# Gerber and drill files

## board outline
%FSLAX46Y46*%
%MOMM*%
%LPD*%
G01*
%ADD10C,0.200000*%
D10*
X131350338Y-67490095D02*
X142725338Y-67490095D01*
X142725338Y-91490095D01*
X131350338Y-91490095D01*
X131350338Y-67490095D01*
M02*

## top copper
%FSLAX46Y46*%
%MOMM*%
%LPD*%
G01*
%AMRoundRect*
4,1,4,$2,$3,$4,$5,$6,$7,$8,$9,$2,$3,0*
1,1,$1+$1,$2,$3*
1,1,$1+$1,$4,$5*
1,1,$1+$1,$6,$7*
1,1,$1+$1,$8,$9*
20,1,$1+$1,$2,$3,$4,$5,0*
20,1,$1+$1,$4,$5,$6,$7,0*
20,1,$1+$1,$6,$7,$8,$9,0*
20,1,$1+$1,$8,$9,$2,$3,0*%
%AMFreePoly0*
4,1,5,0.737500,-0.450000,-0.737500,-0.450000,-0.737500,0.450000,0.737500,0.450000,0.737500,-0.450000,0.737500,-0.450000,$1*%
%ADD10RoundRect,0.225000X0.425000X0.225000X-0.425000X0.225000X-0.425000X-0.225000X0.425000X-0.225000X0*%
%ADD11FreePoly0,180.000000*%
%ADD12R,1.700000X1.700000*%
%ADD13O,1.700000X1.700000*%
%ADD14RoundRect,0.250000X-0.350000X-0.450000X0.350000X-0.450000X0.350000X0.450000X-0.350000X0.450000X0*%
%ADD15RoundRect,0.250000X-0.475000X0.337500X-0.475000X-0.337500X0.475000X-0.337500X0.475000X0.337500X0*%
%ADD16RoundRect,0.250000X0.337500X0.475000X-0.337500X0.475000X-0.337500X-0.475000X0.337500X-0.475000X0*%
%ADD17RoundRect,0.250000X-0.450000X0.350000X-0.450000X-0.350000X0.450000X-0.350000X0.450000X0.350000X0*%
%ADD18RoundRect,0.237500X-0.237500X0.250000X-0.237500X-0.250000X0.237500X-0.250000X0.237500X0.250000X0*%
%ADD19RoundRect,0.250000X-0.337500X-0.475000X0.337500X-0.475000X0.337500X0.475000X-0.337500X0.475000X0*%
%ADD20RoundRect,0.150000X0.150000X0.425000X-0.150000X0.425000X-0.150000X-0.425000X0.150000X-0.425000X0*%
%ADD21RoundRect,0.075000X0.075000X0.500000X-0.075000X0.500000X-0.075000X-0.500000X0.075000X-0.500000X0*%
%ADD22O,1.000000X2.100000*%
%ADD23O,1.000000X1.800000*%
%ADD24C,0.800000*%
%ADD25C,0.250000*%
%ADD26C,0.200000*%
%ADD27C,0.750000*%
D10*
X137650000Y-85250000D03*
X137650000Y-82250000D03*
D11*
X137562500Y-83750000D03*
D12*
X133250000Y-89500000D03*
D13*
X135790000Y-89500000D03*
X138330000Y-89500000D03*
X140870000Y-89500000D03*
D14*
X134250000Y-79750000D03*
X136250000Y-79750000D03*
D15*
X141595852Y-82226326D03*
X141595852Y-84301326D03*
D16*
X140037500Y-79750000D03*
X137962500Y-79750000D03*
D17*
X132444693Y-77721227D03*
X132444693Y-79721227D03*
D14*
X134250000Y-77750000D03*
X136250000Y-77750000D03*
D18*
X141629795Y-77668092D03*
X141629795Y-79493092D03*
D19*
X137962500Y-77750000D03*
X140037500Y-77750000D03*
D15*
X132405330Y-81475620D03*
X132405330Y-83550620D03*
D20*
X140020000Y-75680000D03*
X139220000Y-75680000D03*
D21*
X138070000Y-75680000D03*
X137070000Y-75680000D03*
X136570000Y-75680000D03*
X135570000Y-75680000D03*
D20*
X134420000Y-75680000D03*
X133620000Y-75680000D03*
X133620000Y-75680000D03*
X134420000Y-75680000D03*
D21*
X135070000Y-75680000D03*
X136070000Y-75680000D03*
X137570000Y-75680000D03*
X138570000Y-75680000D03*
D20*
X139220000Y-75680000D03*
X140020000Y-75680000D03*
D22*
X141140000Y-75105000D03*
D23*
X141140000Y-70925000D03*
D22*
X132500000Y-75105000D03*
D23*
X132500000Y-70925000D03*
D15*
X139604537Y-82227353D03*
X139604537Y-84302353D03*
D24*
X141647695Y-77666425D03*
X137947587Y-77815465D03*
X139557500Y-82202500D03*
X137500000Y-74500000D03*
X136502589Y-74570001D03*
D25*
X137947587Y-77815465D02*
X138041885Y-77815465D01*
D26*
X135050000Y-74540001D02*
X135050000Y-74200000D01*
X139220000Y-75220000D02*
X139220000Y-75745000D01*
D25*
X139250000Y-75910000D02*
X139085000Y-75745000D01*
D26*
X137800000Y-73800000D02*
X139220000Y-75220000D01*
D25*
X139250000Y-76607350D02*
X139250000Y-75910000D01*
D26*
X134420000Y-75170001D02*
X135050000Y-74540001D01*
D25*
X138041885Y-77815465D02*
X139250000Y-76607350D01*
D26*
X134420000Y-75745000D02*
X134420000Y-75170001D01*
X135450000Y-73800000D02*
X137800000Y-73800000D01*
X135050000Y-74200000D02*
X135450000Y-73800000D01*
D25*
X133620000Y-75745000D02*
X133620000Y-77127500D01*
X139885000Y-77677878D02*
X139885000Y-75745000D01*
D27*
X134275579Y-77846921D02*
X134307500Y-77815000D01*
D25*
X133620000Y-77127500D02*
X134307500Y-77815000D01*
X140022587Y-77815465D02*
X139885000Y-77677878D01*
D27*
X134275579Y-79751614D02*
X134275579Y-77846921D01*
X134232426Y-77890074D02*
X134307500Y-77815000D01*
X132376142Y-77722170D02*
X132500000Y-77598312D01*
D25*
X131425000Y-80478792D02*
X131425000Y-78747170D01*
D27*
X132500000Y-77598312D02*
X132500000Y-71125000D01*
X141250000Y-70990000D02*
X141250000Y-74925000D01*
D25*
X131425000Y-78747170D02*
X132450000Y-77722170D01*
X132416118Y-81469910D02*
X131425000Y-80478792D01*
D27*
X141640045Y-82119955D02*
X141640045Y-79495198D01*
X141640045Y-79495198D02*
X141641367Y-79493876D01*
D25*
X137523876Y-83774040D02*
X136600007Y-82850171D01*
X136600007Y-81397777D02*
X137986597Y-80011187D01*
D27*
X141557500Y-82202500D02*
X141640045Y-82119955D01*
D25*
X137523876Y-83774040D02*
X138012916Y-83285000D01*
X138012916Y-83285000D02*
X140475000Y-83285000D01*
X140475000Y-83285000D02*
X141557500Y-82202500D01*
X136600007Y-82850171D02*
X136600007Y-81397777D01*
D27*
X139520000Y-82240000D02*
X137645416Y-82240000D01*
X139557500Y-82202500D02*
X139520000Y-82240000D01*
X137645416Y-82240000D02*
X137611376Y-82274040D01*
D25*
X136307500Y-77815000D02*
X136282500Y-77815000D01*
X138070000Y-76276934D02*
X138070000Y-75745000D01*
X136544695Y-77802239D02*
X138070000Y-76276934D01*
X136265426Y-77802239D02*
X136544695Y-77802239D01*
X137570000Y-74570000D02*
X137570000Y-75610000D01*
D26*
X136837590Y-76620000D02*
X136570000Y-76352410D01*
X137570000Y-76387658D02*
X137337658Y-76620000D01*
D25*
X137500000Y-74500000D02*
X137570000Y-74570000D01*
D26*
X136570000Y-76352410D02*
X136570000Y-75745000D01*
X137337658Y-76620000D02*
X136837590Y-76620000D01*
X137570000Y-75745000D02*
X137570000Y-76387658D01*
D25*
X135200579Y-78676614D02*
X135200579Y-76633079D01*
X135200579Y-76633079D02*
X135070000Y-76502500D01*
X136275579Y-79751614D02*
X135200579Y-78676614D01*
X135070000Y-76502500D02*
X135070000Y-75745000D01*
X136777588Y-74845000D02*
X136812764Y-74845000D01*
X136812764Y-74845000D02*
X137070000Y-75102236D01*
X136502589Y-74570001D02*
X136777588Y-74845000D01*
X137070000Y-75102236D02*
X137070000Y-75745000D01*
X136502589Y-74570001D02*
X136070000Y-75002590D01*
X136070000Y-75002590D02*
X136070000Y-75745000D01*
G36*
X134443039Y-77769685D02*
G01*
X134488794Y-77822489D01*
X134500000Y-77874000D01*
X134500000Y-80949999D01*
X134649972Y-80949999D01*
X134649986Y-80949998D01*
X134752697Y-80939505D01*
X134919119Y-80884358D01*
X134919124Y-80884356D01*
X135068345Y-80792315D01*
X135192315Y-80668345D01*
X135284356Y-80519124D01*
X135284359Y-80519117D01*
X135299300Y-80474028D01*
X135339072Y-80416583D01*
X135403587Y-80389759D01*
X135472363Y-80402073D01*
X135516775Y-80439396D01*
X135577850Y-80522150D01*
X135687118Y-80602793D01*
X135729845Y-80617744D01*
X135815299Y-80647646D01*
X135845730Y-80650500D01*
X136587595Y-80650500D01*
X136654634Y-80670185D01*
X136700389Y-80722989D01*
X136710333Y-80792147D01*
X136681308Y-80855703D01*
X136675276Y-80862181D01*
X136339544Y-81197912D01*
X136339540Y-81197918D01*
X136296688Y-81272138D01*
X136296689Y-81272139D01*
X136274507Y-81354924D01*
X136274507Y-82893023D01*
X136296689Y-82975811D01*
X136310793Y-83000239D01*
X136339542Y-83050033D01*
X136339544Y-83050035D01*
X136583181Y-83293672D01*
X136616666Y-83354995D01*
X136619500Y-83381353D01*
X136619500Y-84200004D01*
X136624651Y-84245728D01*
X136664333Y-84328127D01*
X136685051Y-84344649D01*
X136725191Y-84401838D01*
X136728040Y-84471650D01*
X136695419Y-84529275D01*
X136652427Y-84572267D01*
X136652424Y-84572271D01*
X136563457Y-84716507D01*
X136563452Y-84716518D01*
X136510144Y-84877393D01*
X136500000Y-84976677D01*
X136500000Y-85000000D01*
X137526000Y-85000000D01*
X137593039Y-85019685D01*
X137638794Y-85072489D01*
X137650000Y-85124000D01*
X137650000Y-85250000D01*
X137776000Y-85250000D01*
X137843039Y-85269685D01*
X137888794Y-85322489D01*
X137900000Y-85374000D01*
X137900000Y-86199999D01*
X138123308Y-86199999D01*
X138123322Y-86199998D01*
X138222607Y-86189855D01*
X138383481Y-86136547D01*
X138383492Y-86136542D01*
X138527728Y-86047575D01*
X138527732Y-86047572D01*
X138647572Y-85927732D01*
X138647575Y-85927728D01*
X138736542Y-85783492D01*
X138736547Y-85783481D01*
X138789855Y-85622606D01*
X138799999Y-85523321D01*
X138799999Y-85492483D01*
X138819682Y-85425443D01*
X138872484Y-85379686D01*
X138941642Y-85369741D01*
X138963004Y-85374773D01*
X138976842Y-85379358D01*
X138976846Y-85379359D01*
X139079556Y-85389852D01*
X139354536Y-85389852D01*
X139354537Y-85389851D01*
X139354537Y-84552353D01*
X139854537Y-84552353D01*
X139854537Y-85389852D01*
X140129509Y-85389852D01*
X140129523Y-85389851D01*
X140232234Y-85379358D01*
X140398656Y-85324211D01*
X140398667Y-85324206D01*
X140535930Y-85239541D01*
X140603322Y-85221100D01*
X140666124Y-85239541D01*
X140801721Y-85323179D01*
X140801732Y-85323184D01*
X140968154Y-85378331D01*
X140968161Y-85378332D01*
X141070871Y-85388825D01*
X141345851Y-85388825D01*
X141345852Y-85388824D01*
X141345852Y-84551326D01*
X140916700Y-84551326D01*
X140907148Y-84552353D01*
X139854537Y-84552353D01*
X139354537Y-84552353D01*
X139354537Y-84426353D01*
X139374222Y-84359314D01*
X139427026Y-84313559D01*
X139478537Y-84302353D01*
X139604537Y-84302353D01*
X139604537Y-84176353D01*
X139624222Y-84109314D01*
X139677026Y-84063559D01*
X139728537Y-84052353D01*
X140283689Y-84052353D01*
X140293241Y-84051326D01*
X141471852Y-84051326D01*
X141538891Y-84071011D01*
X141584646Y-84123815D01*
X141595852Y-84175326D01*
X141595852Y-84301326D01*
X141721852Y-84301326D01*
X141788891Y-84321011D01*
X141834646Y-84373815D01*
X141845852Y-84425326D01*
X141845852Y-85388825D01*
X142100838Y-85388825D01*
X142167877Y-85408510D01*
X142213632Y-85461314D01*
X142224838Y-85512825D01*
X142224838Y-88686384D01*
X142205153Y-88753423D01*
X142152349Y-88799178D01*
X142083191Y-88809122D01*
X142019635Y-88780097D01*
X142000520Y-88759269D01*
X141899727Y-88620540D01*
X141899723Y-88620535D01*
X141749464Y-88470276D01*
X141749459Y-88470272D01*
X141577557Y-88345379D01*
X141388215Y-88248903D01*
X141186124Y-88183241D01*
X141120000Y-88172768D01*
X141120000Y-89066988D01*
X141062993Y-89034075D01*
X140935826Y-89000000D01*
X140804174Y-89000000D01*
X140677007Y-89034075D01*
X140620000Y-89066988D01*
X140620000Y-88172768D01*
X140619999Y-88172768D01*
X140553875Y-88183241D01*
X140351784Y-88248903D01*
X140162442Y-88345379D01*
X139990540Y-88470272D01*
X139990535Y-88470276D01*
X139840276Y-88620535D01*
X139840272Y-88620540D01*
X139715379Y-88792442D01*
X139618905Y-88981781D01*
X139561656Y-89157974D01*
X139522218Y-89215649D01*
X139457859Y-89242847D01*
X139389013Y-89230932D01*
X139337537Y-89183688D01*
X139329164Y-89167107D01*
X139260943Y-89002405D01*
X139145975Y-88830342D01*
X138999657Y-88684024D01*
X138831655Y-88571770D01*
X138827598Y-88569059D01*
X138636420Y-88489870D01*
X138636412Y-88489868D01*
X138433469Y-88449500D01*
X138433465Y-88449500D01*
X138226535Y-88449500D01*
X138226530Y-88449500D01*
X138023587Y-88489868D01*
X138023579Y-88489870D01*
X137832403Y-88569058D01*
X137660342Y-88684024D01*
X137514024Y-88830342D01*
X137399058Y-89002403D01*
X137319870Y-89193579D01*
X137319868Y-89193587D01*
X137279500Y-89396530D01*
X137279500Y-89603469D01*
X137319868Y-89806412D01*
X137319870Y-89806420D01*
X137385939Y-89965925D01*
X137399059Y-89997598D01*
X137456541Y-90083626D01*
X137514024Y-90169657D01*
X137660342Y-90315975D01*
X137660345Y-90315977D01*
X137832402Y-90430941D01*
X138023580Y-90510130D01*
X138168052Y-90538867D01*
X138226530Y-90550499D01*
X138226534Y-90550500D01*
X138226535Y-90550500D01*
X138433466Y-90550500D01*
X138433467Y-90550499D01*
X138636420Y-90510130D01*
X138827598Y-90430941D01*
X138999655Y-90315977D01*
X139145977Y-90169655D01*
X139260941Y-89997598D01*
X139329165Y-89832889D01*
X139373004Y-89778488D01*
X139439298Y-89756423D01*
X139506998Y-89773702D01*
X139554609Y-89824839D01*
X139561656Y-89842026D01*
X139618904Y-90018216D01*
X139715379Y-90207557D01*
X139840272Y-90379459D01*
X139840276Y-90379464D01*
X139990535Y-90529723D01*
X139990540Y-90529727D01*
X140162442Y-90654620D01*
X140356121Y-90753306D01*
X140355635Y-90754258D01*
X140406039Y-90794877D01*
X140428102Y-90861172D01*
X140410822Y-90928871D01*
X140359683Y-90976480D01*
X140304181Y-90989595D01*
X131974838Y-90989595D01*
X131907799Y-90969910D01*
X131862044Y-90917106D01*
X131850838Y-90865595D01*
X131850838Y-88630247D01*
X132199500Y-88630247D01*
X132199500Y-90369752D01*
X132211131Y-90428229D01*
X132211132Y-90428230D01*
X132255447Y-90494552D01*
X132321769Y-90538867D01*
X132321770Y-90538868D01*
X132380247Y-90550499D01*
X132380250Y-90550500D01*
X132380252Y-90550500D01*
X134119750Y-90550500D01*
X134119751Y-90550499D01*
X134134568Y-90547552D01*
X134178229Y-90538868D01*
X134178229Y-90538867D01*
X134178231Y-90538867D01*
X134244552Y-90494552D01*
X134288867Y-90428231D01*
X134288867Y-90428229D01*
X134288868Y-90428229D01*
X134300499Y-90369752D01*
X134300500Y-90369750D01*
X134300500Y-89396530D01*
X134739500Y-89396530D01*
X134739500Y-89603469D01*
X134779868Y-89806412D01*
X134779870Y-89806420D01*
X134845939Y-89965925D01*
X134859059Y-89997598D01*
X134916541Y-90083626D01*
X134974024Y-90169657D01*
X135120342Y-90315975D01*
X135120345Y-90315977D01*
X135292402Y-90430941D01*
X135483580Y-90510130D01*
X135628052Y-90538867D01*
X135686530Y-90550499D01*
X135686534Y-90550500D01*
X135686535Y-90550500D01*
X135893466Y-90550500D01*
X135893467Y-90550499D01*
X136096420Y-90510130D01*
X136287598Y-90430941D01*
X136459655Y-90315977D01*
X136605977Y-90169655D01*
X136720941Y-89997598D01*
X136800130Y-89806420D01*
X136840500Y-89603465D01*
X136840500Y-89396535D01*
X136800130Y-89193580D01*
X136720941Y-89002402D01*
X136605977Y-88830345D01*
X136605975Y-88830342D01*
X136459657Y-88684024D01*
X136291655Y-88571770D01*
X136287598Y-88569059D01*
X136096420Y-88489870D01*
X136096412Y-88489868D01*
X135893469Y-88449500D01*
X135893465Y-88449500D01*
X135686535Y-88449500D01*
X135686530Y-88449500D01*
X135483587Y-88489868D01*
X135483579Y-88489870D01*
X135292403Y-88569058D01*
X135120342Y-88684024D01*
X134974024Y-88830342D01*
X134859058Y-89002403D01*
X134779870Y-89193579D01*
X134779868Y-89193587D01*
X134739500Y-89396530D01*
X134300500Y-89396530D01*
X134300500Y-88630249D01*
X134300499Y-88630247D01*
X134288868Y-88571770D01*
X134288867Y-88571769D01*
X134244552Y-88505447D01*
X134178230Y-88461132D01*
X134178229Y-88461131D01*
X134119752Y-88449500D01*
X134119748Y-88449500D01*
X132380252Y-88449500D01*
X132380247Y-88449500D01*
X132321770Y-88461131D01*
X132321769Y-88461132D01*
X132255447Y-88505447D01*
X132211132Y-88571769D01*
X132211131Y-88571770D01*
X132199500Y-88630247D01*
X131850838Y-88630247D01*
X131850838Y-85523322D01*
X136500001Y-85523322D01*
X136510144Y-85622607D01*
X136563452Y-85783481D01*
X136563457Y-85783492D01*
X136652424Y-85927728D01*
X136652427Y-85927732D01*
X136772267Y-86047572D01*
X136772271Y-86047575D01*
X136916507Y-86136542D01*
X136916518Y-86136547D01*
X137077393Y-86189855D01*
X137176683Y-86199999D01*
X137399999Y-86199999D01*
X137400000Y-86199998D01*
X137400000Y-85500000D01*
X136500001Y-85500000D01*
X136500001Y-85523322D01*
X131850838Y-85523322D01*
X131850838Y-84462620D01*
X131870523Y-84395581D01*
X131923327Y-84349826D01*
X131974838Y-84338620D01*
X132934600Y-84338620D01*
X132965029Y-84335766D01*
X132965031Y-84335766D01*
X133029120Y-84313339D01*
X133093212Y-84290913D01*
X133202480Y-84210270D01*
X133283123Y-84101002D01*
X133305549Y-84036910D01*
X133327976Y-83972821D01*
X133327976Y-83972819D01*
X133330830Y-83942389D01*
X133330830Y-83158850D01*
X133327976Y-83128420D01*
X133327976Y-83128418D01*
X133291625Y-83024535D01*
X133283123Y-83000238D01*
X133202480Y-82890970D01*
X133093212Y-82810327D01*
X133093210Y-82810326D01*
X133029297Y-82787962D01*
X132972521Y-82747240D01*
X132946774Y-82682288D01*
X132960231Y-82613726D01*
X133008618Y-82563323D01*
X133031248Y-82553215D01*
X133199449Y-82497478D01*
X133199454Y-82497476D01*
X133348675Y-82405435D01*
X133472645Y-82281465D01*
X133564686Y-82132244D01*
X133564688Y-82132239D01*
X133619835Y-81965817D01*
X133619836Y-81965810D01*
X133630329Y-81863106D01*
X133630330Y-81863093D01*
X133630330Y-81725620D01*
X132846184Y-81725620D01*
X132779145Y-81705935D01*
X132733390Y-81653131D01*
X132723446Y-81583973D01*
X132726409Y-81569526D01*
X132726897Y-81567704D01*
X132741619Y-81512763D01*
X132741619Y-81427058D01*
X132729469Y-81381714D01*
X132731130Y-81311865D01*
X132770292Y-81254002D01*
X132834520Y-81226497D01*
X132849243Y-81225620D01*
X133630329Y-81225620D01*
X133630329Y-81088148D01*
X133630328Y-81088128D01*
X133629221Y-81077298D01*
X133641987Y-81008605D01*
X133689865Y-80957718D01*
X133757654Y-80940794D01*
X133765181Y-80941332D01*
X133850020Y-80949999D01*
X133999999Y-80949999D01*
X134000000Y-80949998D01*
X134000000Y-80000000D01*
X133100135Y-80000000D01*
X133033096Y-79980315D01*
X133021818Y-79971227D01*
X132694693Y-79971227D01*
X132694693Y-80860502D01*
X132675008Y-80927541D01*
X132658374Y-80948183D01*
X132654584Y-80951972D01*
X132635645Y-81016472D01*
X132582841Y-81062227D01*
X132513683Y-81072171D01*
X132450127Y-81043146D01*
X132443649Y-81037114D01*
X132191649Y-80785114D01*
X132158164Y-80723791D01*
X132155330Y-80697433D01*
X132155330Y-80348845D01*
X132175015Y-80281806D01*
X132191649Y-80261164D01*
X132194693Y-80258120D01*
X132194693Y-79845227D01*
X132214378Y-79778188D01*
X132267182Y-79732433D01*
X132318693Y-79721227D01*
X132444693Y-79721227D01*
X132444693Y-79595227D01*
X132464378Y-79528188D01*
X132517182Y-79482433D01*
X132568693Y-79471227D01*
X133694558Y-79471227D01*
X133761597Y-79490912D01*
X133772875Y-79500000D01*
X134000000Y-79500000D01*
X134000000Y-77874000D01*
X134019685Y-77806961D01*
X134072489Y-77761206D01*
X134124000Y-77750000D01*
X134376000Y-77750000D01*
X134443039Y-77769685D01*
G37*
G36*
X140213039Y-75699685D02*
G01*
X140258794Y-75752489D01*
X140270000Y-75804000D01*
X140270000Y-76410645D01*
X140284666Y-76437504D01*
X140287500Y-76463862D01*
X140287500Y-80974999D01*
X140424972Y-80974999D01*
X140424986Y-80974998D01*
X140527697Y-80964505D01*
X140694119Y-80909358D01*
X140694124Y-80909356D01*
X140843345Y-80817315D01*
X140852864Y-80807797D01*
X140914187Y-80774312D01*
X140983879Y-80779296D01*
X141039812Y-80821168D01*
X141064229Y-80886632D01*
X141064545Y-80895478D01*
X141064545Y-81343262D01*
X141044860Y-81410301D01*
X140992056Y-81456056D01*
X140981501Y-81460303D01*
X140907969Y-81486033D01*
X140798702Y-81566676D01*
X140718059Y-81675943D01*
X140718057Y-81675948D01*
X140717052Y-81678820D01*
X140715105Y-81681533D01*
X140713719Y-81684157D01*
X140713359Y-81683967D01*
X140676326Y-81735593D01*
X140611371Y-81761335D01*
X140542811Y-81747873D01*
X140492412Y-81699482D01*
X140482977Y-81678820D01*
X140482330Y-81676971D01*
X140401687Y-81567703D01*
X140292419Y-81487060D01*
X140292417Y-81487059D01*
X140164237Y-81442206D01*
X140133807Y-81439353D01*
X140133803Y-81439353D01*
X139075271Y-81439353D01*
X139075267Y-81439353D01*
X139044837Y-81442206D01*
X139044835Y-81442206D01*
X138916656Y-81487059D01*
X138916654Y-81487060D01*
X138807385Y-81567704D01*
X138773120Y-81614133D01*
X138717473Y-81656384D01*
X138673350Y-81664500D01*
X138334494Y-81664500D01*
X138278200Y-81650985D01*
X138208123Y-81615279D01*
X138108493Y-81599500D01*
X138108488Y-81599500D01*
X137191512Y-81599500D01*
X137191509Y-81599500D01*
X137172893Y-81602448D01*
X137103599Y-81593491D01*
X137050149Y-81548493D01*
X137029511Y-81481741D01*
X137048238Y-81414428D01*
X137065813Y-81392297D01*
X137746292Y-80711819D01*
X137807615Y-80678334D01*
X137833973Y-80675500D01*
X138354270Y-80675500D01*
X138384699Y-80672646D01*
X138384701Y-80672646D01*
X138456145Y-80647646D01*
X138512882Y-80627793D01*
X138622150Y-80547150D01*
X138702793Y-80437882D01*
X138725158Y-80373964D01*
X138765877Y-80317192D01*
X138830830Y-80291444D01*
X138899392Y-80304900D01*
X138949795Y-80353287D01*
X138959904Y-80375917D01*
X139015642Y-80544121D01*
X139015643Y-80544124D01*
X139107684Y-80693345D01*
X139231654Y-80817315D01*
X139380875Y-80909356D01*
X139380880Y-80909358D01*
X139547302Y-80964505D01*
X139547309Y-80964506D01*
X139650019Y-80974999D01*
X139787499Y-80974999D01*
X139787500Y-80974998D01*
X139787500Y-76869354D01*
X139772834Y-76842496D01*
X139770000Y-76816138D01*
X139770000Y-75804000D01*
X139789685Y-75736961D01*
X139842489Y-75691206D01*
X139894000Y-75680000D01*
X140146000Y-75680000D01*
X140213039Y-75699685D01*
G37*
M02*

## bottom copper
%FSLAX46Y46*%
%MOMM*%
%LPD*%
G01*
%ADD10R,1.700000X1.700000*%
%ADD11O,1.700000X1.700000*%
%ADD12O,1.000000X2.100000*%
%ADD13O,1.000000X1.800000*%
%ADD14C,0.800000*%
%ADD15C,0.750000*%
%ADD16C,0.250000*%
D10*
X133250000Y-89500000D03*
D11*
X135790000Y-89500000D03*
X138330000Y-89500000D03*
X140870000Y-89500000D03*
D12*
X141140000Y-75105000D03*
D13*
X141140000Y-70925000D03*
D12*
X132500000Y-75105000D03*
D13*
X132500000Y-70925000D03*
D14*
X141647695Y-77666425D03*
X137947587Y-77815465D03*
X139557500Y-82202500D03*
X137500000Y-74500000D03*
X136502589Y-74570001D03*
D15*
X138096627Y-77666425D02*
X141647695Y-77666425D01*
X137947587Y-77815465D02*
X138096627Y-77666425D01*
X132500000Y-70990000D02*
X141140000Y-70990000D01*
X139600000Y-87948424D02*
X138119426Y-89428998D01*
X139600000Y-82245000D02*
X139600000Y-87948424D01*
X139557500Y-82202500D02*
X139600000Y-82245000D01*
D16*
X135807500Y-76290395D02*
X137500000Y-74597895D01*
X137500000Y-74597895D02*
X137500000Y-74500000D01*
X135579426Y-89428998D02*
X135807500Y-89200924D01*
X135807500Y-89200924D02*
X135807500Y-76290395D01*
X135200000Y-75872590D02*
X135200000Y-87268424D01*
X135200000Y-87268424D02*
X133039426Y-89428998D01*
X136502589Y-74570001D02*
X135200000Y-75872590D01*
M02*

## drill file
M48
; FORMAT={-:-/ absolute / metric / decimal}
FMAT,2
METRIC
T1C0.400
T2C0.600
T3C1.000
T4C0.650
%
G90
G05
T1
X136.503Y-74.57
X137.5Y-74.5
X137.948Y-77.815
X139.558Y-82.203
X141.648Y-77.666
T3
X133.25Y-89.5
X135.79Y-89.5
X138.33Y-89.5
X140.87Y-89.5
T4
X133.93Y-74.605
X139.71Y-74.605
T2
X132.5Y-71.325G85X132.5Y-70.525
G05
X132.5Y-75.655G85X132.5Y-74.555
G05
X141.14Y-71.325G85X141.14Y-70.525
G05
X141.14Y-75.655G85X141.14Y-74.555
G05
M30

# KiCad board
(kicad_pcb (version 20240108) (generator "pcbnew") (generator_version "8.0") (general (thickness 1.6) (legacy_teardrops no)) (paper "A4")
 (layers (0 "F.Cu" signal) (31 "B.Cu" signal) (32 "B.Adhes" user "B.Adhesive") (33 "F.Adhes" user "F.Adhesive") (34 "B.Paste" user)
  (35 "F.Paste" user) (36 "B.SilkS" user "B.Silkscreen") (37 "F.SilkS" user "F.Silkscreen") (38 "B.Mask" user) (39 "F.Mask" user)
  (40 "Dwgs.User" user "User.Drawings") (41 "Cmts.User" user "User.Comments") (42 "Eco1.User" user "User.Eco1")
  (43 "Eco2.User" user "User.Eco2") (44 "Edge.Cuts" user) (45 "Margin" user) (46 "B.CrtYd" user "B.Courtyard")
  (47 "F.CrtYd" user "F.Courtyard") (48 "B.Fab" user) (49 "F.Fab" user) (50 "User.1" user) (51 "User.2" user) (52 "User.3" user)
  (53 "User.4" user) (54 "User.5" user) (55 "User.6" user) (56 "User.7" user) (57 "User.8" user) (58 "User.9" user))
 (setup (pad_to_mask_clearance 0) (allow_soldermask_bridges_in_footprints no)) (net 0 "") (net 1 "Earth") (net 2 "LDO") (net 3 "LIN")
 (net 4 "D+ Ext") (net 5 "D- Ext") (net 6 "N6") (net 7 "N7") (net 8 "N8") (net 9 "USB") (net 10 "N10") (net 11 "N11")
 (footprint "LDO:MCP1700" (layer "F.Cu") (at 136 83.75 180)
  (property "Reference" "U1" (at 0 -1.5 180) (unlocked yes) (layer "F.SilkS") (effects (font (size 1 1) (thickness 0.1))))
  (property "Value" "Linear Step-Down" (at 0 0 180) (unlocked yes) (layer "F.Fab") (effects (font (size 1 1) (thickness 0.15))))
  (pad "1" smd roundrect (at -1.65 -1.5 180) (size 1.3 0.9) (layers "F.Cu" "F.Paste" "F.Mask") (roundrect_rratio 0.25) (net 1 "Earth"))
  (pad "2" smd roundrect (at -1.65 1.5 180) (size 1.3 0.9) (layers "F.Cu" "F.Paste" "F.Mask") (roundrect_rratio 0.25) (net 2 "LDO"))
  (pad "3" smd custom (at -1.5625 0 180) (size 1.475 0.9) (layers "F.Cu" "F.Paste" "F.Mask") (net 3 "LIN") (zone_connect 2)
   (thermal_bridge_angle 45) (options (clearance outline) (anchor rect)) (primitives)))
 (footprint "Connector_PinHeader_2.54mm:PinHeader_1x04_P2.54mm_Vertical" (layer "F.Cu") (at 133.25 89.5 90)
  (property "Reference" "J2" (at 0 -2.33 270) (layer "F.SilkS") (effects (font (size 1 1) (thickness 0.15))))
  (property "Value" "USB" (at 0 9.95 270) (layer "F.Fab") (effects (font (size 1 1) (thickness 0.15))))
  (pad "1" thru_hole rect (at 0 0 90) (size 1.7 1.7) (drill 1) (layers "*.Cu" "*.Mask") (remove_unused_layers no) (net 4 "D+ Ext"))
  (pad "2" thru_hole oval (at 0 2.54 90) (size 1.7 1.7) (drill 1) (layers "*.Cu" "*.Mask") (remove_unused_layers no) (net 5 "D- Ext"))
  (pad "3" thru_hole oval (at 0 5.08 90) (size 1.7 1.7) (drill 1) (layers "*.Cu" "*.Mask") (remove_unused_layers no) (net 2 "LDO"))
  (pad "4" thru_hole oval (at 0 7.62 90) (size 1.7 1.7) (drill 1) (layers "*.Cu" "*.Mask") (remove_unused_layers no) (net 1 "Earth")))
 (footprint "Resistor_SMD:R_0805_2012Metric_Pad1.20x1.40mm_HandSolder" (layer "F.Cu") (at 135.25 79.75)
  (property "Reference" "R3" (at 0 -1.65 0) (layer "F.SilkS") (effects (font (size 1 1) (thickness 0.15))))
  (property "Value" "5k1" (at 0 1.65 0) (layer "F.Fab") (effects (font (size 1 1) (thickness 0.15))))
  (pad "1" smd roundrect (at -1 0) (size 1.2 1.4) (layers "F.Cu" "F.Paste" "F.Mask") (roundrect_rratio 0.208333) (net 1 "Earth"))
  (pad "2" smd roundrect (at 1 0) (size 1.2 1.4) (layers "F.Cu" "F.Paste" "F.Mask") (roundrect_rratio 0.208333) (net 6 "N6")))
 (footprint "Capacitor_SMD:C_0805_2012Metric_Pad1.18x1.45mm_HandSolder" (layer "F.Cu") (at 141.595852 83.263826 -90)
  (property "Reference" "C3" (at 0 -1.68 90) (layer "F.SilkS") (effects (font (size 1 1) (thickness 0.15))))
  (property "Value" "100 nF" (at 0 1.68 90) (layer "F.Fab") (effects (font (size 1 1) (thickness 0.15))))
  (pad "1" smd roundrect (at -1.0375 0 270) (size 1.175 1.45) (layers "F.Cu" "F.Paste" "F.Mask") (roundrect_rratio 0.212766) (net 3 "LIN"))
  (pad "2" smd roundrect (at 1.0375 0 270) (size 1.175 1.45) (layers "F.Cu" "F.Paste" "F.Mask") (roundrect_rratio 0.212766) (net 1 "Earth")))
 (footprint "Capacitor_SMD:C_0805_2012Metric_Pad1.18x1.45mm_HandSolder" (layer "F.Cu") (at 139 79.75 180)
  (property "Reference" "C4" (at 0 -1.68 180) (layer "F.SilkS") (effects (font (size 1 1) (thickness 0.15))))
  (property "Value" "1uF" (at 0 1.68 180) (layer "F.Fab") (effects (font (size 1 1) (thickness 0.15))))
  (pad "1" smd roundrect (at -1.0375 0 180) (size 1.175 1.45) (layers "F.Cu" "F.Paste" "F.Mask") (roundrect_rratio 0.212766) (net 1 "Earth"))
  (pad "2" smd roundrect (at 1.0375 0 180) (size 1.175 1.45) (layers "F.Cu" "F.Paste" "F.Mask") (roundrect_rratio 0.212766) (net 3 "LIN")))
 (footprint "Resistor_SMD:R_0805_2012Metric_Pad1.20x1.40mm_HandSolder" (layer "F.Cu") (at 132.444693 78.721227 -90)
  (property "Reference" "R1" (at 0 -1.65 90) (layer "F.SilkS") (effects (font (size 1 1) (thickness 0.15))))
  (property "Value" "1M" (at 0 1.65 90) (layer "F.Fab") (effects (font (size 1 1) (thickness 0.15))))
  (pad "1" smd roundrect (at -1 0 270) (size 1.2 1.4) (layers "F.Cu" "F.Paste" "F.Mask") (roundrect_rratio 0.208333) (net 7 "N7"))
  (pad "2" smd roundrect (at 1 0 270) (size 1.2 1.4) (layers "F.Cu" "F.Paste" "F.Mask") (roundrect_rratio 0.208333) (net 1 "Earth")))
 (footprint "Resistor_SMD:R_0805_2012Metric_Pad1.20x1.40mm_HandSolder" (layer "F.Cu") (at 135.25 77.75)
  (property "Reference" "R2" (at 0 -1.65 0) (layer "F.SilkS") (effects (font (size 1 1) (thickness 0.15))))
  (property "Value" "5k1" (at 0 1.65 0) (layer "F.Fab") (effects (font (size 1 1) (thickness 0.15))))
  (pad "1" smd roundrect (at -1 0) (size 1.2 1.4) (layers "F.Cu" "F.Paste" "F.Mask") (roundrect_rratio 0.208333) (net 1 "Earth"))
  (pad "2" smd roundrect (at 1 0) (size 1.2 1.4) (layers "F.Cu" "F.Paste" "F.Mask") (roundrect_rratio 0.208333) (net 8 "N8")))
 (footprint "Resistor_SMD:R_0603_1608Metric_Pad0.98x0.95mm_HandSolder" (layer "F.Cu") (at 141.629795 78.580592 -90)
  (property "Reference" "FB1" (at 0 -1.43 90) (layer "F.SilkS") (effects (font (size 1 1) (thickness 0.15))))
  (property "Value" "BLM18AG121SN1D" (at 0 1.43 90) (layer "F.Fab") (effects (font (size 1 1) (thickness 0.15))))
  (pad "1" smd roundrect (at -0.9125 0 270) (size 0.975 0.95) (layers "F.Cu" "F.Paste" "F.Mask") (roundrect_rratio 0.25) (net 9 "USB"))
  (pad "2" smd roundrect (at 0.9125 0 270) (size 0.975 0.95) (layers "F.Cu" "F.Paste" "F.Mask") (roundrect_rratio 0.25) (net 3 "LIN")))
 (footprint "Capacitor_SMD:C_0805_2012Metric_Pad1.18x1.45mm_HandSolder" (layer "F.Cu") (at 139 77.75)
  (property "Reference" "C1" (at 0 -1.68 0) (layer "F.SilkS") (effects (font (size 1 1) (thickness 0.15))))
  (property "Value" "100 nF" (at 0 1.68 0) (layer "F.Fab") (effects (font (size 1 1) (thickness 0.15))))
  (pad "1" smd roundrect (at -1.0375 0) (size 1.175 1.45) (layers "F.Cu" "F.Paste" "F.Mask") (roundrect_rratio 0.212766) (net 9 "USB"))
  (pad "2" smd roundrect (at 1.0375 0) (size 1.175 1.45) (layers "F.Cu" "F.Paste" "F.Mask") (roundrect_rratio 0.212766) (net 1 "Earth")))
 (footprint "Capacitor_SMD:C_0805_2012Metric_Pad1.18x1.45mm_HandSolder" (layer "F.Cu") (at 132.40533 82.51312 -90)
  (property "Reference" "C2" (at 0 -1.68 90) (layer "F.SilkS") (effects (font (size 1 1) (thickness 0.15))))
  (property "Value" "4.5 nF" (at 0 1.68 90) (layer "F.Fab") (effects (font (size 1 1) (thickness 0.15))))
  (pad "1" smd roundrect (at -1.0375 0 270) (size 1.175 1.45) (layers "F.Cu" "F.Paste" "F.Mask") (roundrect_rratio 0.212766) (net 1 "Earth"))
  (pad "2" smd roundrect (at 1.0375 0 270) (size 1.175 1.45) (layers "F.Cu" "F.Paste" "F.Mask") (roundrect_rratio 0.212766) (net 7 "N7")))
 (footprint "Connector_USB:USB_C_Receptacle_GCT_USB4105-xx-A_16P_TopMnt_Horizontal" (layer "F.Cu") (at 136.82 72 180)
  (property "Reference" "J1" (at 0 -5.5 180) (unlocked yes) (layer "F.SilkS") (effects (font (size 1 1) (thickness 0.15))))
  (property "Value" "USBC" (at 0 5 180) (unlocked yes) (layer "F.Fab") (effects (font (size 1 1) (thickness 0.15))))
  (pad "" np_thru_hole circle (at -2.89 -2.605 180) (size 0.65 0.65) (drill 0.65) (layers "F&B.Cu" "*.Mask"))
  (pad "" np_thru_hole circle (at 2.89 -2.605 180) (size 0.65 0.65) (drill 0.65) (layers "F&B.Cu" "*.Mask"))
  (pad "A1" smd roundrect (at -3.2 -3.68 180) (size 0.6 1.15) (layers "F.Cu" "F.Paste" "F.Mask") (roundrect_rratio 0.25) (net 1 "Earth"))
  (pad "A4" smd roundrect (at -2.4 -3.68 180) (size 0.6 1.15) (layers "F.Cu" "F.Paste" "F.Mask") (roundrect_rratio 0.25) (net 9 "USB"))
  (pad "A5" smd roundrect (at -1.25 -3.68 180) (size 0.3 1.15) (layers "F.Cu" "F.Paste" "F.Mask") (roundrect_rratio 0.25) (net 8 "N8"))
  (pad "A6" smd roundrect (at -0.25 -3.68 180) (size 0.3 1.15) (layers "F.Cu" "F.Paste" "F.Mask") (roundrect_rratio 0.25) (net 4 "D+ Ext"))
  (pad "A7" smd roundrect (at 0.25 -3.68 180) (size 0.3 1.15) (layers "F.Cu" "F.Paste" "F.Mask") (roundrect_rratio 0.25) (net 5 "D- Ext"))
  (pad "A8" smd roundrect (at 1.25 -3.68 180) (size 0.3 1.15) (layers "F.Cu" "F.Paste" "F.Mask") (roundrect_rratio 0.25) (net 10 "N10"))
  (pad "A9" smd roundrect (at 2.4 -3.68 180) (size 0.6 1.15) (layers "F.Cu" "F.Paste" "F.Mask") (roundrect_rratio 0.25) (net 9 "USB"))
  (pad "A12" smd roundrect (at 3.2 -3.68 180) (size 0.6 1.15) (layers "F.Cu" "F.Paste" "F.Mask") (roundrect_rratio 0.25) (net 1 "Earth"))
  (pad "B1" smd roundrect (at 3.2 -3.68 180) (size 0.6 1.15) (layers "F.Cu" "F.Paste" "F.Mask") (roundrect_rratio 0.25) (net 1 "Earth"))
  (pad "B4" smd roundrect (at 2.4 -3.68 180) (size 0.6 1.15) (layers "F.Cu" "F.Paste" "F.Mask") (roundrect_rratio 0.25) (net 9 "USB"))
  (pad "B5" smd roundrect (at 1.75 -3.68 180) (size 0.3 1.15) (layers "F.Cu" "F.Paste" "F.Mask") (roundrect_rratio 0.25) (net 6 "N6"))
  (pad "B6" smd roundrect (at 0.75 -3.68 180) (size 0.3 1.15) (layers "F.Cu" "F.Paste" "F.Mask") (roundrect_rratio 0.25) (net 4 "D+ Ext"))
  (pad "B7" smd roundrect (at -0.75 -3.68 180) (size 0.3 1.15) (layers "F.Cu" "F.Paste" "F.Mask") (roundrect_rratio 0.25) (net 5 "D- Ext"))
  (pad "B8" smd roundrect (at -1.75 -3.68 180) (size 0.3 1.15) (layers "F.Cu" "F.Paste" "F.Mask") (roundrect_rratio 0.25) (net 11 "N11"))
  (pad "B9" smd roundrect (at -2.4 -3.68 180) (size 0.6 1.15) (layers "F.Cu" "F.Paste" "F.Mask") (roundrect_rratio 0.25) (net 9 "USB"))
  (pad "B12" smd roundrect (at -3.2 -3.68 180) (size 0.6 1.15) (layers "F.Cu" "F.Paste" "F.Mask") (roundrect_rratio 0.25) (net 1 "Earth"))
  (pad "S1" thru_hole oval (at -4.32 -3.105 180) (size 1 2.1) (drill oval 0.6 1.7) (layers "*.Cu" "*.Mask" "F.Paste")
   (remove_unused_layers no) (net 7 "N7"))
  (pad "S1" thru_hole oval (at -4.32 1.075 180) (size 1 1.8) (drill oval 0.6 1.4) (layers "*.Cu" "*.Mask" "F.Paste")
   (remove_unused_layers no) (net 7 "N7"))
  (pad "S1" thru_hole oval (at 4.32 -3.105 180) (size 1 2.1) (drill oval 0.6 1.7) (layers "*.Cu" "*.Mask" "F.Paste")
   (remove_unused_layers no) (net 7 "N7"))
  (pad "S1" thru_hole oval (at 4.32 1.075 180) (size 1 1.8) (drill oval 0.6 1.4) (layers "*.Cu" "*.Mask" "F.Paste")
   (remove_unused_layers no) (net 7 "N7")))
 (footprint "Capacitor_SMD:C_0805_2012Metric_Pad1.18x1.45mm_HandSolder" (layer "F.Cu") (at 139.604537 83.264853 -90)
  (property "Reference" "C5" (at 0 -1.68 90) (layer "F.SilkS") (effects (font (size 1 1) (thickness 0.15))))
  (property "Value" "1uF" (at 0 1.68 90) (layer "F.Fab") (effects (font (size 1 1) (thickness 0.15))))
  (pad "1" smd roundrect (at -1.0375 0 270) (size 1.175 1.45) (layers "F.Cu" "F.Paste" "F.Mask") (roundrect_rratio 0.212766) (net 2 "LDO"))
  (pad "2" smd roundrect (at 1.0375 0 270) (size 1.175 1.45) (layers "F.Cu" "F.Paste" "F.Mask") (roundrect_rratio 0.212766) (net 1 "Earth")))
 (gr_rect (start 131.350338 67.490095) (end 142.725338 91.490095) (stroke (width 0.2) (type default)) (fill none) (layer "Edge.Cuts"))
 (segment (start 137.947587 77.815465) (end 138.041885 77.815465) (width 0.25) (layer "F.Cu") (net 9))
 (segment (start 135.05 74.540001) (end 135.05 74.2) (width 0.2) (layer "F.Cu") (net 9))
 (segment (start 139.22 75.22) (end 139.22 75.745) (width 0.2) (layer "F.Cu") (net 9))
 (segment (start 139.25 75.91) (end 139.085 75.745) (width 0.25) (layer "F.Cu") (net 9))
 (segment (start 137.8 73.8) (end 139.22 75.22) (width 0.2) (layer "F.Cu") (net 9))
 (segment (start 139.25 76.60735) (end 139.25 75.91) (width 0.25) (layer "F.Cu") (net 9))
 (segment (start 134.42 75.170001) (end 135.05 74.540001) (width 0.2) (layer "F.Cu") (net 9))
 (segment (start 138.041885 77.815465) (end 139.25 76.60735) (width 0.25) (layer "F.Cu") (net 9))
 (segment (start 134.42 75.745) (end 134.42 75.170001) (width 0.2) (layer "F.Cu") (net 9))
 (segment (start 135.45 73.8) (end 137.8 73.8) (width 0.2) (layer "F.Cu") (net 9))
 (segment (start 135.05 74.2) (end 135.45 73.8) (width 0.2) (layer "F.Cu") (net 9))
 (via (at 141.647695 77.666425) (size 0.8) (drill 0.4) (layers "F.Cu" "B.Cu") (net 9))
 (via (at 137.947587 77.815465) (size 0.8) (drill 0.4) (layers "F.Cu" "B.Cu") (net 9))
 (segment (start 138.096627 77.666425) (end 141.647695 77.666425) (width 0.75) (layer "B.Cu") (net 9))
 (segment (start 137.947587 77.815465) (end 138.096627 77.666425) (width 0.75) (layer "B.Cu") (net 9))
 (segment (start 133.62 75.745) (end 133.62 77.1275) (width 0.25) (layer "F.Cu") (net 1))
 (segment (start 139.885 77.677878) (end 139.885 75.745) (width 0.25) (layer "F.Cu") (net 1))
 (segment (start 134.275579 77.846921) (end 134.3075 77.815) (width 0.75) (layer "F.Cu") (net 1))
 (segment (start 133.62 77.1275) (end 134.3075 77.815) (width 0.25) (layer "F.Cu") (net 1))
 (segment (start 140.022587 77.815465) (end 139.885 77.677878) (width 0.25) (layer "F.Cu") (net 1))
 (segment (start 134.275579 79.751614) (end 134.275579 77.846921) (width 0.75) (layer "F.Cu") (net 1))
 (segment (start 134.232426 77.890074) (end 134.3075 77.815) (width 0.75) (layer "F.Cu") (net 1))
 (segment (start 132.376142 77.72217) (end 132.5 77.598312) (width 0.75) (layer "F.Cu") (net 7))
 (segment (start 131.425 80.478792) (end 131.425 78.74717) (width 0.25) (layer "F.Cu") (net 7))
 (segment (start 132.5 77.598312) (end 132.5 71.125) (width 0.75) (layer "F.Cu") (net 7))
 (segment (start 141.25 70.99) (end 141.25 74.925) (width 0.75) (layer "F.Cu") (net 7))
 (segment (start 131.425 78.74717) (end 132.45 77.72217) (width 0.25) (layer "F.Cu") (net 7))
 (segment (start 132.416118 81.46991) (end 131.425 80.478792) (width 0.25) (layer "F.Cu") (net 7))
 (segment (start 132.5 70.99) (end 141.14 70.99) (width 0.75) (layer "B.Cu") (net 7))
 (segment (start 141.640045 82.119955) (end 141.640045 79.495198) (width 0.75) (layer "F.Cu") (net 3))
 (segment (start 141.640045 79.495198) (end 141.641367 79.493876) (width 0.75) (layer "F.Cu") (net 3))
 (segment (start 137.523876 83.77404) (end 136.600007 82.850171) (width 0.25) (layer "F.Cu") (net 3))
 (segment (start 136.600007 81.397777) (end 137.986597 80.011187) (width 0.25) (layer "F.Cu") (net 3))
 (segment (start 141.5575 82.2025) (end 141.640045 82.119955) (width 0.75) (layer "F.Cu") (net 3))
 (segment (start 137.523876 83.77404) (end 138.012916 83.285) (width 0.25) (layer "F.Cu") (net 3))
 (segment (start 138.012916 83.285) (end 140.475 83.285) (width 0.25) (layer "F.Cu") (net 3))
 (segment (start 140.475 83.285) (end 141.5575 82.2025) (width 0.25) (layer "F.Cu") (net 3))
 (segment (start 136.600007 82.850171) (end 136.600007 81.397777) (width 0.25) (layer "F.Cu") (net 3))
 (segment (start 139.52 82.24) (end 137.645416 82.24) (width 0.75) (layer "F.Cu") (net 2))
 (segment (start 139.5575 82.2025) (end 139.52 82.24) (width 0.75) (layer "F.Cu") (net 2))
 (segment (start 137.645416 82.24) (end 137.611376 82.27404) (width 0.75) (layer "F.Cu") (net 2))
 (via (at 139.5575 82.2025) (size 0.8) (drill 0.4) (layers "F.Cu" "B.Cu") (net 2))
 (segment (start 139.6 87.948424) (end 138.119426 89.428998) (width 0.75) (layer "B.Cu") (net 2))
 (segment (start 139.6 82.245) (end 139.6 87.948424) (width 0.75) (layer "B.Cu") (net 2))
 (segment (start 139.5575 82.2025) (end 139.6 82.245) (width 0.75) (layer "B.Cu") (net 2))
 (segment (start 136.3075 77.815) (end 136.2825 77.815) (width 0.25) (layer "F.Cu") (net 8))
 (segment (start 138.07 76.276934) (end 138.07 75.745) (width 0.25) (layer "F.Cu") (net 8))
 (segment (start 136.544695 77.802239) (end 138.07 76.276934) (width 0.25) (layer "F.Cu") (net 8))
 (segment (start 136.265426 77.802239) (end 136.544695 77.802239) (width 0.25) (layer "F.Cu") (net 8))
 (segment (start 137.57 74.57) (end 137.57 75.61) (width 0.25) (layer "F.Cu") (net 5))
 (segment (start 136.83759 76.62) (end 136.57 76.35241) (width 0.2) (layer "F.Cu") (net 5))
 (segment (start 137.57 76.387658) (end 137.337658 76.62) (width 0.2) (layer "F.Cu") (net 5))
 (segment (start 137.5 74.5) (end 137.57 74.57) (width 0.25) (layer "F.Cu") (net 5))
 (segment (start 136.57 76.35241) (end 136.57 75.745) (width 0.2) (layer "F.Cu") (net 5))
 (segment (start 137.337658 76.62) (end 136.83759 76.62) (width 0.2) (layer "F.Cu") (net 5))
 (segment (start 137.57 75.745) (end 137.57 76.387658) (width 0.2) (layer "F.Cu") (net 5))
 (via (at 137.5 74.5) (size 0.8) (drill 0.4) (layers "F.Cu" "B.Cu") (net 5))
 (segment (start 135.8075 76.290395) (end 137.5 74.597895) (width 0.25) (layer "B.Cu") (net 5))
 (segment (start 137.5 74.597895) (end 137.5 74.5) (width 0.25) (layer "B.Cu") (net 5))
 (segment (start 135.579426 89.428998) (end 135.8075 89.200924) (width 0.25) (layer "B.Cu") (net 5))
 (segment (start 135.8075 89.200924) (end 135.8075 76.290395) (width 0.25) (layer "B.Cu") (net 5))
 (segment (start 135.200579 78.676614) (end 135.200579 76.633079) (width 0.25) (layer "F.Cu") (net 6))
 (segment (start 135.200579 76.633079) (end 135.07 76.5025) (width 0.25) (layer "F.Cu") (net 6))
 (segment (start 136.275579 79.751614) (end 135.200579 78.676614) (width 0.25) (layer "F.Cu") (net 6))
 (segment (start 135.07 76.5025) (end 135.07 75.745) (width 0.25) (layer "F.Cu") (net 6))
 (segment (start 136.777588 74.845) (end 136.812764 74.845) (width 0.25) (layer "F.Cu") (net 4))
 (segment (start 136.812764 74.845) (end 137.07 75.102236) (width 0.25) (layer "F.Cu") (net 4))
 (segment (start 136.502589 74.570001) (end 136.777588 74.845) (width 0.25) (layer "F.Cu") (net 4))
 (segment (start 137.07 75.102236) (end 137.07 75.745) (width 0.25) (layer "F.Cu") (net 4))
 (segment (start 136.502589 74.570001) (end 136.07 75.00259) (width 0.25) (layer "F.Cu") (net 4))
 (segment (start 136.07 75.00259) (end 136.07 75.745) (width 0.25) (layer "F.Cu") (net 4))
 (via (at 136.502589 74.570001) (size 0.8) (drill 0.4) (layers "F.Cu" "B.Cu") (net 4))
 (segment (start 135.2 75.87259) (end 135.2 87.268424) (width 0.25) (layer "B.Cu") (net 4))
 (segment (start 135.2 87.268424) (end 133.039426 89.428998) (width 0.25) (layer "B.Cu") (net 4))
 (segment (start 136.502589 74.570001) (end 135.2 75.87259) (width 0.25) (layer "B.Cu") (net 4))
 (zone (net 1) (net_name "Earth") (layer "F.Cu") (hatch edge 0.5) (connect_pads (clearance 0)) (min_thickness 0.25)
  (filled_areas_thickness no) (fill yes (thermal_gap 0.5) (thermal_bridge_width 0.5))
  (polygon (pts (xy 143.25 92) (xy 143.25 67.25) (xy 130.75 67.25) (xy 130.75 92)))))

